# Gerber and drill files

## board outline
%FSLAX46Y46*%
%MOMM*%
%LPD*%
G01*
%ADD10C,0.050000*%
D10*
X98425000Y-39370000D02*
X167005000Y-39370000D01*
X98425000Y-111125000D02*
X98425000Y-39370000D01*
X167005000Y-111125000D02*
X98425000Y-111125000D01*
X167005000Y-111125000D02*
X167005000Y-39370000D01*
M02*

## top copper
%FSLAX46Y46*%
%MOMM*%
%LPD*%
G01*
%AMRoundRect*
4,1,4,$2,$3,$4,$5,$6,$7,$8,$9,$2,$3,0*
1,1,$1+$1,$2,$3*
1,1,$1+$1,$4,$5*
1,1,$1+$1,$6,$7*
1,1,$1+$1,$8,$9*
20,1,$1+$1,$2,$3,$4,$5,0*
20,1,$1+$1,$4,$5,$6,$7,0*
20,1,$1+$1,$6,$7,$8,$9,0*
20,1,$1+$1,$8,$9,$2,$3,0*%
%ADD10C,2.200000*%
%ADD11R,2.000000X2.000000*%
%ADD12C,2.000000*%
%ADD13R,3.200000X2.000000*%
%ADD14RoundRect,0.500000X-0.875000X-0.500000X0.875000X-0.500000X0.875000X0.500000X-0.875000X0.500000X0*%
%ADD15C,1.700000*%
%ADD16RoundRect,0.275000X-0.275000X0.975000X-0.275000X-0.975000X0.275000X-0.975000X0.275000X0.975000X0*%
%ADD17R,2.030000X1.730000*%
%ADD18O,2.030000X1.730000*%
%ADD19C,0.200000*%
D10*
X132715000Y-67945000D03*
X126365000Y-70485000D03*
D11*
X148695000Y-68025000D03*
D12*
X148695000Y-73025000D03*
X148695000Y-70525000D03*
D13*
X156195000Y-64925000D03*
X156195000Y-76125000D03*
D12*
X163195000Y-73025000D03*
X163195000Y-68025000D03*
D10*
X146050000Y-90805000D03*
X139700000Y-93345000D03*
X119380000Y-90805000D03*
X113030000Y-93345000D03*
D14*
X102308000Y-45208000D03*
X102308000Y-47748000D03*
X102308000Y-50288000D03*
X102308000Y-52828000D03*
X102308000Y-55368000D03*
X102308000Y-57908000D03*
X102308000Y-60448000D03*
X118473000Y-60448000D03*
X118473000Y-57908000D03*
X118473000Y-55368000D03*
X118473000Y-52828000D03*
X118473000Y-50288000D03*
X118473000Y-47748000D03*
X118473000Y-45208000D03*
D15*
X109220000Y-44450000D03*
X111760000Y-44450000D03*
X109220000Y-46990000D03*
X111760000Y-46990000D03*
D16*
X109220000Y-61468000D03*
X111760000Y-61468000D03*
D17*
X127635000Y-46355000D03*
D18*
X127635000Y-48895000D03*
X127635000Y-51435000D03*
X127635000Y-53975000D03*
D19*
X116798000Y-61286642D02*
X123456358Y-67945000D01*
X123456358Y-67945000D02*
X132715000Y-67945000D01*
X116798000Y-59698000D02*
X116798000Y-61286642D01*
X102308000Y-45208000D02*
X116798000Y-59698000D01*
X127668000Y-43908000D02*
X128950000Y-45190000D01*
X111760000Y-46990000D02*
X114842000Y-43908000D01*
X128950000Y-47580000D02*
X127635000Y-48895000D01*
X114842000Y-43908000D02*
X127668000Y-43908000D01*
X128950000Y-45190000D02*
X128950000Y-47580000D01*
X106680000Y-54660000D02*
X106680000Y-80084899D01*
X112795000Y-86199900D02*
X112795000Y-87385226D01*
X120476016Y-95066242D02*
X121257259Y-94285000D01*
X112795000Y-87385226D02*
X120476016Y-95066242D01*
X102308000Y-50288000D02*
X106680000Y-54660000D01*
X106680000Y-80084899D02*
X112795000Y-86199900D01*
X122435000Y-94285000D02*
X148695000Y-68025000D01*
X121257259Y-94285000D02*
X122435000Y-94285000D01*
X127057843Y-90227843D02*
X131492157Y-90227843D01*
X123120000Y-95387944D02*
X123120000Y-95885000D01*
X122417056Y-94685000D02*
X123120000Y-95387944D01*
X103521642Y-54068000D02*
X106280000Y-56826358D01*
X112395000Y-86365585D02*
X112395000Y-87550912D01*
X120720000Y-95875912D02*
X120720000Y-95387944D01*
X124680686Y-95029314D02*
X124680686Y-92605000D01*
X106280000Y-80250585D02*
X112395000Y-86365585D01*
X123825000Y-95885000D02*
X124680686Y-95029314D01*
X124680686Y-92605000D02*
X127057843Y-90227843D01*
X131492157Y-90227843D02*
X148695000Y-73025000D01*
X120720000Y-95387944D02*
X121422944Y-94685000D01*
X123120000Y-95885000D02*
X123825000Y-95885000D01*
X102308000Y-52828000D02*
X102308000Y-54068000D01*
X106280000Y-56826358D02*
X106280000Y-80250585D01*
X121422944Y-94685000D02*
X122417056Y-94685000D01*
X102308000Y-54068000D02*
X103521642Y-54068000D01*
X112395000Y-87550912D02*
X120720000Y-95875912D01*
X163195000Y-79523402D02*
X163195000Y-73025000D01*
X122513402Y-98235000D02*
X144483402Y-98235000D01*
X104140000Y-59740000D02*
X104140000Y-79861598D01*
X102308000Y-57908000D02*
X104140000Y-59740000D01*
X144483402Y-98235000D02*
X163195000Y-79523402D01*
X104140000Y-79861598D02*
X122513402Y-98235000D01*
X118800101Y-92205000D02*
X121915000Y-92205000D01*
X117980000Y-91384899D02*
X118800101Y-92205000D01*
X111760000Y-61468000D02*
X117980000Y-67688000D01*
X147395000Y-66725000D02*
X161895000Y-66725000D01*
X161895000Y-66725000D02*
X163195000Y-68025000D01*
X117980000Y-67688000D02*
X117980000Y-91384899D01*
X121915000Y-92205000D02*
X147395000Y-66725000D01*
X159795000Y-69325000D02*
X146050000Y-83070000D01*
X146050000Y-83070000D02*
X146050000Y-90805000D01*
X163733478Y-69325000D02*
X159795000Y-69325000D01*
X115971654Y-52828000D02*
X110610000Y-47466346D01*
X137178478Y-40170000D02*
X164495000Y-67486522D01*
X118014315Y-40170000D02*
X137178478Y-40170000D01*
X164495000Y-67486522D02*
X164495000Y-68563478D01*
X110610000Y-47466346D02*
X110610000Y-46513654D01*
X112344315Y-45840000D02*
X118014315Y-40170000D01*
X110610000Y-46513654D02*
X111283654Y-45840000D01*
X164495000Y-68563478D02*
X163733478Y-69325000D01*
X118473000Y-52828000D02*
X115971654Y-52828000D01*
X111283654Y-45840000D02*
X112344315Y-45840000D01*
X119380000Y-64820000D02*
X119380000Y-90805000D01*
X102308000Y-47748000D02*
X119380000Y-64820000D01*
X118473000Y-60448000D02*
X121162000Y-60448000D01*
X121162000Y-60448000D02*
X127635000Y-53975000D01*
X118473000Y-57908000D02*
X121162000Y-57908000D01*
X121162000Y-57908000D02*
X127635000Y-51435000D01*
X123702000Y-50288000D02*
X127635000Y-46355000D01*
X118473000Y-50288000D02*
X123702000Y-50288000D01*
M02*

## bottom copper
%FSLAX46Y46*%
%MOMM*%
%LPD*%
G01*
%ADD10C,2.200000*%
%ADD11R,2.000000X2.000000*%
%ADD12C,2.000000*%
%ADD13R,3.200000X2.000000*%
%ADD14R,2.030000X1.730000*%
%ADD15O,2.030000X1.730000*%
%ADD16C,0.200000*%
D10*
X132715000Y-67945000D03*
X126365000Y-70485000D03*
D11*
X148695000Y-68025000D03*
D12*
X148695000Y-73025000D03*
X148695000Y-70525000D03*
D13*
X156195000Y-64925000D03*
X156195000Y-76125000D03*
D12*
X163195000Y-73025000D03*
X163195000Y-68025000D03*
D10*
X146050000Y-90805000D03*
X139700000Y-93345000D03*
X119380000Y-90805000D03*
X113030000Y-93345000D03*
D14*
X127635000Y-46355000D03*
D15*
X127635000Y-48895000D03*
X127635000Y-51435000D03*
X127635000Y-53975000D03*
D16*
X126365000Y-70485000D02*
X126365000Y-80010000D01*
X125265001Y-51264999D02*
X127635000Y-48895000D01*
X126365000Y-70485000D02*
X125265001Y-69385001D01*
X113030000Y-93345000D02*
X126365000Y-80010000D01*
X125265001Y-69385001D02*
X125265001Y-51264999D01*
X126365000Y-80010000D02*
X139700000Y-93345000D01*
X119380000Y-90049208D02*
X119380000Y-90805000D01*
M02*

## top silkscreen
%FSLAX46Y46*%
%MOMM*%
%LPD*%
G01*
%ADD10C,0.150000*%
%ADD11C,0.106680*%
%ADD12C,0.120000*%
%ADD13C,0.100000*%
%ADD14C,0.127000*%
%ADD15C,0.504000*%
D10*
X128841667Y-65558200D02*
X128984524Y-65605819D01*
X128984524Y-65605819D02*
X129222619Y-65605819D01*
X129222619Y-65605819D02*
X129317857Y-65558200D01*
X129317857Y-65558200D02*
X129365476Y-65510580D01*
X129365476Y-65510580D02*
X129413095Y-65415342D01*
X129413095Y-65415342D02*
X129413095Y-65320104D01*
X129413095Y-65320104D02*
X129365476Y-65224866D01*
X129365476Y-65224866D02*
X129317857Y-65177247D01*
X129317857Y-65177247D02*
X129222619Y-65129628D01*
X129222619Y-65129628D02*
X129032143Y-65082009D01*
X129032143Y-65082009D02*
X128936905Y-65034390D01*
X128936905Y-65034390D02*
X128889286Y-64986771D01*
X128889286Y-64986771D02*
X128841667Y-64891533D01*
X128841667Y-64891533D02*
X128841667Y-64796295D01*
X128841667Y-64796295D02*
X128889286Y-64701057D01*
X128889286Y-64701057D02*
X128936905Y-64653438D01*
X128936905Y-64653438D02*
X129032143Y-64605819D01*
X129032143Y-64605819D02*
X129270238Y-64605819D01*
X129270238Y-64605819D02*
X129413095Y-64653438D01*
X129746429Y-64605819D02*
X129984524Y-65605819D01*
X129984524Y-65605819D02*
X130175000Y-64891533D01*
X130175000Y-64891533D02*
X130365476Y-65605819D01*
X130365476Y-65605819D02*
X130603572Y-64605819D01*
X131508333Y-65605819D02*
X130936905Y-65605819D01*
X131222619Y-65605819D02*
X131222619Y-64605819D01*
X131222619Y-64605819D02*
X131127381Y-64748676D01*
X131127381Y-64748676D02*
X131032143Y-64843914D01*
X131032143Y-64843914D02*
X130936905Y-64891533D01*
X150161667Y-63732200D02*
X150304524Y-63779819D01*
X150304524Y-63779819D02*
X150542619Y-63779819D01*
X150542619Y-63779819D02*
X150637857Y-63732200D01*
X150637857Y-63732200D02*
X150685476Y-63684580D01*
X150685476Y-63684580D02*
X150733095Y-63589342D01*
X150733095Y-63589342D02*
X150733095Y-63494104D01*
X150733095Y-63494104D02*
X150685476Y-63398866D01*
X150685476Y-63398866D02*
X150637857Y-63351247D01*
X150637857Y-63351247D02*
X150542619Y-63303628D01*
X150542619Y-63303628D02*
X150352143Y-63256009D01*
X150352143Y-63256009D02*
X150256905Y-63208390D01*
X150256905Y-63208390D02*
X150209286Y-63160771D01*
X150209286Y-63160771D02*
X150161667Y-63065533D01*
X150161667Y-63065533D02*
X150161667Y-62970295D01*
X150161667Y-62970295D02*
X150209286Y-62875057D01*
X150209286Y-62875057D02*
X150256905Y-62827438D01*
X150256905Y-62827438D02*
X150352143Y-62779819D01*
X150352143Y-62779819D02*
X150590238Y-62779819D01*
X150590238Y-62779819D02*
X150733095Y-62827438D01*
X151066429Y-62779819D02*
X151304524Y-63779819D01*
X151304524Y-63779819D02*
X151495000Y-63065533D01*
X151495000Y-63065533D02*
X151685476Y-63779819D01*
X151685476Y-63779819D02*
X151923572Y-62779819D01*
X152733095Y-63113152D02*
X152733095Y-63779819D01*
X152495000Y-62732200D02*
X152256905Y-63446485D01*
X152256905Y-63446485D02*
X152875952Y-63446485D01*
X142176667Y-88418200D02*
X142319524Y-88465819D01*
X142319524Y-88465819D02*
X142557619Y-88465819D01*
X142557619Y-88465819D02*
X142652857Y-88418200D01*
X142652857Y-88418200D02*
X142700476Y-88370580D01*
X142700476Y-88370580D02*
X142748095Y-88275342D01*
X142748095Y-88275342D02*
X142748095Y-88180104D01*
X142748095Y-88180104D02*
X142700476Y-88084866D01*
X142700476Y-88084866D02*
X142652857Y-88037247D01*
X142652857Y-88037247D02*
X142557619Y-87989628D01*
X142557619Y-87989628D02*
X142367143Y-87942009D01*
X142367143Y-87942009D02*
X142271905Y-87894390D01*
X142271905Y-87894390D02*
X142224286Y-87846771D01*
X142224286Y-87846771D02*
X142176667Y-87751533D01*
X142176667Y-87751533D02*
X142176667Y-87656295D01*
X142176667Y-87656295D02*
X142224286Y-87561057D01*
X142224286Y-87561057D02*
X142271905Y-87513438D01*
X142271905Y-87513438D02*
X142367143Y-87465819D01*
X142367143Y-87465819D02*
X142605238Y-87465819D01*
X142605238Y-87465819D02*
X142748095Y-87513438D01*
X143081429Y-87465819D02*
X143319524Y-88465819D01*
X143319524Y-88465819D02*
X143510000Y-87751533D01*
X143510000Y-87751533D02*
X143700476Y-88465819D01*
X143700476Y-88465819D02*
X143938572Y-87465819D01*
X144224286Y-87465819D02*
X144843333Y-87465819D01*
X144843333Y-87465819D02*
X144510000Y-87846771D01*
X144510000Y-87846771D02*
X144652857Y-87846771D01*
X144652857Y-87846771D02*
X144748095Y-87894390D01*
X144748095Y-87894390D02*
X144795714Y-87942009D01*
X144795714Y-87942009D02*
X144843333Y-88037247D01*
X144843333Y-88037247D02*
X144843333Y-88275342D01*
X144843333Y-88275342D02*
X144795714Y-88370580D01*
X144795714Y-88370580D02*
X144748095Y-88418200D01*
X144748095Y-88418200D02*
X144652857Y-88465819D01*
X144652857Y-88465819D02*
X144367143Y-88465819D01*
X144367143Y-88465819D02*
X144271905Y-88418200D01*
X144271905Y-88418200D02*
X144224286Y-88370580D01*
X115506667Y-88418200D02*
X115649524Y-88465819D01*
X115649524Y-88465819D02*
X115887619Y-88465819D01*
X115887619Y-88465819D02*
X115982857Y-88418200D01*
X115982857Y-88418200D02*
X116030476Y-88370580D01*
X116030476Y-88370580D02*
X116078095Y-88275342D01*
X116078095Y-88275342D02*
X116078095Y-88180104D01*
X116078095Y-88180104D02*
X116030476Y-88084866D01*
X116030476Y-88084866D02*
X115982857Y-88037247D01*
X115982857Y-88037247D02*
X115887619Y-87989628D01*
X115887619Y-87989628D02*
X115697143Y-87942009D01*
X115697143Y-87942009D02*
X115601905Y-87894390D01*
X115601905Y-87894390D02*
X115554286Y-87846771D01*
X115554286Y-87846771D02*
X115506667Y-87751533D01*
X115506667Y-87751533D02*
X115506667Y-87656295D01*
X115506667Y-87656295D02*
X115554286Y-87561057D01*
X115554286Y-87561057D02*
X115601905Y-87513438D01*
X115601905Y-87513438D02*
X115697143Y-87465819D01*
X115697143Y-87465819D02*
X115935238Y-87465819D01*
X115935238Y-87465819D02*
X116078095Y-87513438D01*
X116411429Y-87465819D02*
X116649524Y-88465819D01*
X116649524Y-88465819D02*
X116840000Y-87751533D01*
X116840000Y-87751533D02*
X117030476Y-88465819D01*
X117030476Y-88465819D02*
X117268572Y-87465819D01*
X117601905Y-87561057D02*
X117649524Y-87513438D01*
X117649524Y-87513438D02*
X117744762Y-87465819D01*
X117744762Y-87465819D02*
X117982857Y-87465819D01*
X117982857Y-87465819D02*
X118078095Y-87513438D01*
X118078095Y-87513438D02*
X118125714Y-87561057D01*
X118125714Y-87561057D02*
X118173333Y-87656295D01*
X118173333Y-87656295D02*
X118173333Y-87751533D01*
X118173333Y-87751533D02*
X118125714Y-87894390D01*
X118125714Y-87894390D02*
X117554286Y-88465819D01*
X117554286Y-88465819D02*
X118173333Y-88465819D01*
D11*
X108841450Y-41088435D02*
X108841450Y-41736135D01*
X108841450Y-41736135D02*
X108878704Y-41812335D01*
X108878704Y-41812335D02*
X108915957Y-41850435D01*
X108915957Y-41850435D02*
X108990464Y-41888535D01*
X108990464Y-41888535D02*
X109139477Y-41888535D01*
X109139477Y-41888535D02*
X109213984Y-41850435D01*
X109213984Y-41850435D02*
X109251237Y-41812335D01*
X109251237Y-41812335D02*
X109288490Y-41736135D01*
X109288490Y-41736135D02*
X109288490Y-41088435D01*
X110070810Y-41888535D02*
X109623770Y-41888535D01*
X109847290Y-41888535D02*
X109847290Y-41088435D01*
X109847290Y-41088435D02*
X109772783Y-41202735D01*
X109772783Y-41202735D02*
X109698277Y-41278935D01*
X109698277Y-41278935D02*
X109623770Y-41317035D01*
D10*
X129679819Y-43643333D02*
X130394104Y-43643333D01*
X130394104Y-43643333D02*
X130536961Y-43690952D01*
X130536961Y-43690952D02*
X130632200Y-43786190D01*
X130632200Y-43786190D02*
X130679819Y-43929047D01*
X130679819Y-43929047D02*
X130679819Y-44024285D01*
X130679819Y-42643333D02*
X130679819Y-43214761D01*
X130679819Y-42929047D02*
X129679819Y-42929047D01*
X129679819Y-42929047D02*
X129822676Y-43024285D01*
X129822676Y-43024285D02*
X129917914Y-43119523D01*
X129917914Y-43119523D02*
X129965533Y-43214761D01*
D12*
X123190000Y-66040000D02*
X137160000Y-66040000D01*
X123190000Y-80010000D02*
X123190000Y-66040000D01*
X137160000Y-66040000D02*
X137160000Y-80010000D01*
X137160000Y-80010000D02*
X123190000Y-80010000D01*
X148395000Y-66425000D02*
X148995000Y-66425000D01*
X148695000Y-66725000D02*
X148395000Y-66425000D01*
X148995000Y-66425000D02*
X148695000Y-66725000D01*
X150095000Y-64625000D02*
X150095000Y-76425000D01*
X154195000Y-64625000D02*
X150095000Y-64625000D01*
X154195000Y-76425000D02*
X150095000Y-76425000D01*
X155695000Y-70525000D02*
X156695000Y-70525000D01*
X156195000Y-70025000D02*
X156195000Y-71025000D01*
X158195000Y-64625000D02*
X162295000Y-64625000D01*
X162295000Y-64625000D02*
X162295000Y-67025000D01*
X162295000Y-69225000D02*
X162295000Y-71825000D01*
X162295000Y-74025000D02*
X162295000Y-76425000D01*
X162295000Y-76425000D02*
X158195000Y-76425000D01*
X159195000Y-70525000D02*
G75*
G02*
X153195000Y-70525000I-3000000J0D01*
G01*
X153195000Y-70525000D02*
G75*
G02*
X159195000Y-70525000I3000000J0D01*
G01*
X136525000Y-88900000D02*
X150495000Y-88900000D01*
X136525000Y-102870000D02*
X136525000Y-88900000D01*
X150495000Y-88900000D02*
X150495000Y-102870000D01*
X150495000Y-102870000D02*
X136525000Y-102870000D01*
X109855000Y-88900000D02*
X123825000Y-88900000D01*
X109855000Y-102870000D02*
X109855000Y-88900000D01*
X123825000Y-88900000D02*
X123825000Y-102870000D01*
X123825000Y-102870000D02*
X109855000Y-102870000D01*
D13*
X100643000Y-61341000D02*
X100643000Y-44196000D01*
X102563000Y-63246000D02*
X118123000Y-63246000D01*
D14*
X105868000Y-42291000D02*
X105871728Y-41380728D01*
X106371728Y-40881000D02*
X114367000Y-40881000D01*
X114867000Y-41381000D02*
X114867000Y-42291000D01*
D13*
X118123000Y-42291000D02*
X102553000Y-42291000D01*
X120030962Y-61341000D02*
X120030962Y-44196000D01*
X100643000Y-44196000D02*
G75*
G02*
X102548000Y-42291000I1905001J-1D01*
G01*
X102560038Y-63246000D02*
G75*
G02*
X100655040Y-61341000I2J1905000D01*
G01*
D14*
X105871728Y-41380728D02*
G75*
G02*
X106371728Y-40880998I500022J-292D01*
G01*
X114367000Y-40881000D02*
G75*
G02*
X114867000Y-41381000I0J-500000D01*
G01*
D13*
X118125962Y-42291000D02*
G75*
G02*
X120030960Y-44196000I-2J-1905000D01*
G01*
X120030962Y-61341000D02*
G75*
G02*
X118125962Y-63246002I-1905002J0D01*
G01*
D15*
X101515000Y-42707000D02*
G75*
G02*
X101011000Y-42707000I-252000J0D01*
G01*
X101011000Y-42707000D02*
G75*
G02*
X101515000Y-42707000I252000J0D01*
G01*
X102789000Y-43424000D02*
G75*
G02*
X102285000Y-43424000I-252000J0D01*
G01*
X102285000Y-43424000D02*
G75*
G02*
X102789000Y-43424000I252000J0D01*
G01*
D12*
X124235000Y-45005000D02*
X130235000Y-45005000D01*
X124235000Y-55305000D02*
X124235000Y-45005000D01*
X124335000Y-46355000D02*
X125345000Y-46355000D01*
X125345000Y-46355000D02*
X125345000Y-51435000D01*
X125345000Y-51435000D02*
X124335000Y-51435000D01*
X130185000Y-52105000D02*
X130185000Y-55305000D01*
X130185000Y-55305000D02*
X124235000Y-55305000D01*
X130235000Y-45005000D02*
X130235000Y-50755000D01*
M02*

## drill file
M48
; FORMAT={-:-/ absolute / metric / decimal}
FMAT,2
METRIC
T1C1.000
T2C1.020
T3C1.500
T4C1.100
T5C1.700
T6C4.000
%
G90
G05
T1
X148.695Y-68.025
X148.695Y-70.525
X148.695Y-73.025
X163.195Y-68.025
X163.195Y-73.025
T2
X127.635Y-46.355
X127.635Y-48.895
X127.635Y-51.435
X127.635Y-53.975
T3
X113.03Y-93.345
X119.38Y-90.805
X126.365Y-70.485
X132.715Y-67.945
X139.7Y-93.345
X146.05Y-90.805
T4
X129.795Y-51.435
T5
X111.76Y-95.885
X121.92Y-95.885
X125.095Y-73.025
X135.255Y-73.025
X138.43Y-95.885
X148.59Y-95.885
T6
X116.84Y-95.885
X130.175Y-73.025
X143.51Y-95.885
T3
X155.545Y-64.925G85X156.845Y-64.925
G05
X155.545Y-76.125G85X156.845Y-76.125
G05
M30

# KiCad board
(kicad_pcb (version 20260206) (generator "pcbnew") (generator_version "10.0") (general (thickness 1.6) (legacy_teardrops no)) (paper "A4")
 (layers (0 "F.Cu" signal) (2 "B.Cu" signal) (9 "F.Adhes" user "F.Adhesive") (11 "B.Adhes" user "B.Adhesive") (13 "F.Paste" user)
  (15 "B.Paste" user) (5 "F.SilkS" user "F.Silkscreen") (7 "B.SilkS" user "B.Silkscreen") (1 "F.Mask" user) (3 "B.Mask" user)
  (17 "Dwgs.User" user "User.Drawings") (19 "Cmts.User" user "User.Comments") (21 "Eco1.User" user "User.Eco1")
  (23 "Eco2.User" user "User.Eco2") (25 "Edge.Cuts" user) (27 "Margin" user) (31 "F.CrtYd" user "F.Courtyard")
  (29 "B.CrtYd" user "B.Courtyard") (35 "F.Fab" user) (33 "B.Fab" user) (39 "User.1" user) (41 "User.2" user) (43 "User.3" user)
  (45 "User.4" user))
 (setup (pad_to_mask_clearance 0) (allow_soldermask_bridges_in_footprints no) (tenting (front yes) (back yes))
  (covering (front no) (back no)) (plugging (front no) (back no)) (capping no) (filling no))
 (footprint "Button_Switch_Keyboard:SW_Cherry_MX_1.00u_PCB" (layer "F.Cu") (at 132.715 67.945)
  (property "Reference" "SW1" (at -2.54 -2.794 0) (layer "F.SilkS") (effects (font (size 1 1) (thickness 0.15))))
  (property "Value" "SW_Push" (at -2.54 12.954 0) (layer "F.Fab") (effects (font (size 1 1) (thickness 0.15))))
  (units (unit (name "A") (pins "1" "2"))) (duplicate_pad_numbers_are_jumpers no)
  (fp_line (start -9.525 -1.905) (end 4.445 -1.905) (stroke (width 0.12) (type solid)) (layer "F.SilkS"))
  (fp_line (start -9.525 12.065) (end -9.525 -1.905) (stroke (width 0.12) (type solid)) (layer "F.SilkS"))
  (fp_line (start 4.445 -1.905) (end 4.445 12.065) (stroke (width 0.12) (type solid)) (layer "F.SilkS"))
  (fp_line (start 4.445 12.065) (end -9.525 12.065) (stroke (width 0.12) (type solid)) (layer "F.SilkS"))
  (pad "" np_thru_hole circle (at -7.62 5.08) (size 1.7 1.7) (drill 1.7) (layers "*.Cu" "*.Mask"))
  (pad "" np_thru_hole circle (at -2.54 5.08) (size 4 4) (drill 4) (layers "*.Cu" "*.Mask"))
  (pad "" np_thru_hole circle (at 2.54 5.08) (size 1.7 1.7) (drill 1.7) (layers "*.Cu" "*.Mask"))
  (pad "1" thru_hole circle (at 0 0) (size 2.2 2.2) (drill 1.5) (layers "*.Cu" "*.Mask") (remove_unused_layers no) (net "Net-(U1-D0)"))
  (pad "2" thru_hole circle (at -6.35 2.54) (size 2.2 2.2) (drill 1.5) (layers "*.Cu" "*.Mask") (remove_unused_layers no)
   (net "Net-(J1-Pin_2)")))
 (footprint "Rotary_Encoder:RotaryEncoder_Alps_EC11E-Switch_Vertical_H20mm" (layer "F.Cu") (at 148.695 68.025)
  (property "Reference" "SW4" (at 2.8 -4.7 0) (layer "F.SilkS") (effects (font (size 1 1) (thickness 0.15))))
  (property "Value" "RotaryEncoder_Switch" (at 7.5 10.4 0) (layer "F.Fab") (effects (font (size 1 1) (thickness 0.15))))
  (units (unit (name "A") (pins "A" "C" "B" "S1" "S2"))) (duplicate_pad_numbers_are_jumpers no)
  (fp_line (start -0.3 -1.6) (end 0.3 -1.6) (stroke (width 0.12) (type solid)) (layer "F.SilkS"))
  (fp_line (start 0 -1.3) (end -0.3 -1.6) (stroke (width 0.12) (type solid)) (layer "F.SilkS"))
  (fp_line (start 0.3 -1.6) (end 0 -1.3) (stroke (width 0.12) (type solid)) (layer "F.SilkS"))
  (fp_line (start 1.4 -3.4) (end 1.4 8.4) (stroke (width 0.12) (type solid)) (layer "F.SilkS"))
  (fp_line (start 5.5 -3.4) (end 1.4 -3.4) (stroke (width 0.12) (type solid)) (layer "F.SilkS"))
  (fp_line (start 5.5 8.4) (end 1.4 8.4) (stroke (width 0.12) (type solid)) (layer "F.SilkS"))
  (fp_line (start 7 2.5) (end 8 2.5) (stroke (width 0.12) (type solid)) (layer "F.SilkS"))
  (fp_line (start 7.5 2) (end 7.5 3) (stroke (width 0.12) (type solid)) (layer "F.SilkS"))
  (fp_line (start 9.5 -3.4) (end 13.6 -3.4) (stroke (width 0.12) (type solid)) (layer "F.SilkS"))
  (fp_line (start 13.6 -3.4) (end 13.6 -1) (stroke (width 0.12) (type solid)) (layer "F.SilkS"))
  (fp_line (start 13.6 1.2) (end 13.6 3.8) (stroke (width 0.12) (type solid)) (layer "F.SilkS"))
  (fp_line (start 13.6 6) (end 13.6 8.4) (stroke (width 0.12) (type solid)) (layer "F.SilkS"))
  (fp_line (start 13.6 8.4) (end 9.5 8.4) (stroke (width 0.12) (type solid)) (layer "F.SilkS"))
  (fp_circle (center 7.5 2.5) (end 10.5 2.5) (stroke (width 0.12) (type solid)) (fill no) (layer "F.SilkS"))
  (pad "A" thru_hole rect (at 0 0) (size 2 2) (drill 1) (layers "*.Cu" "*.Mask") (remove_unused_layers no) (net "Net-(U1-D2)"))
  (pad "B" thru_hole circle (at 0 5) (size 2 2) (drill 1) (layers "*.Cu" "*.Mask") (remove_unused_layers no) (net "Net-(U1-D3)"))
  (pad "C" thru_hole circle (at 0 2.5) (size 2 2) (drill 1) (layers "*.Cu" "*.Mask") (remove_unused_layers no)
   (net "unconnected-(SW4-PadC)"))
  (pad "MP" thru_hole rect (at 7.5 -3.1) (size 3.2 2) (drill oval 2.8 1.5) (layers "*.Cu" "*.Mask") (remove_unused_layers no))
  (pad "MP" thru_hole rect (at 7.5 8.1) (size 3.2 2) (drill oval 2.8 1.5) (layers "*.Cu" "*.Mask") (remove_unused_layers no))
  (pad "S1" thru_hole circle (at 14.5 5) (size 2 2) (drill 1) (layers "*.Cu" "*.Mask") (remove_unused_layers no) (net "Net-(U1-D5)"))
  (pad "S2" thru_hole circle (at 14.5 0) (size 2 2) (drill 1) (layers "*.Cu" "*.Mask") (remove_unused_layers no) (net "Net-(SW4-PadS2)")))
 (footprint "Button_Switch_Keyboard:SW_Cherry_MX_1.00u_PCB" (layer "F.Cu") (at 146.05 90.805)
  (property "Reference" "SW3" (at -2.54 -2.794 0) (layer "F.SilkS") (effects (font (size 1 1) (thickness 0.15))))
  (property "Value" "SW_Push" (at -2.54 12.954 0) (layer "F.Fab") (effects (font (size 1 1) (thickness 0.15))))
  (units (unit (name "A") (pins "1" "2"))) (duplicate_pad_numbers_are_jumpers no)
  (fp_line (start -9.525 -1.905) (end 4.445 -1.905) (stroke (width 0.12) (type solid)) (layer "F.SilkS"))
  (fp_line (start -9.525 12.065) (end -9.525 -1.905) (stroke (width 0.12) (type solid)) (layer "F.SilkS"))
  (fp_line (start 4.445 -1.905) (end 4.445 12.065) (stroke (width 0.12) (type solid)) (layer "F.SilkS"))
  (fp_line (start 4.445 12.065) (end -9.525 12.065) (stroke (width 0.12) (type solid)) (layer "F.SilkS"))
  (pad "" np_thru_hole circle (at -7.62 5.08) (size 1.7 1.7) (drill 1.7) (layers "*.Cu" "*.Mask"))
  (pad "" np_thru_hole circle (at -2.54 5.08) (size 4 4) (drill 4) (layers "*.Cu" "*.Mask"))
  (pad "" np_thru_hole circle (at 2.54 5.08) (size 1.7 1.7) (drill 1.7) (layers "*.Cu" "*.Mask"))
  (pad "1" thru_hole circle (at 0 0) (size 2.2 2.2) (drill 1.5) (layers "*.Cu" "*.Mask") (remove_unused_layers no) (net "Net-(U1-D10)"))
  (pad "2" thru_hole circle (at -6.35 2.54) (size 2.2 2.2) (drill 1.5) (layers "*.Cu" "*.Mask") (remove_unused_layers no)
   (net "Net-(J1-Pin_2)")))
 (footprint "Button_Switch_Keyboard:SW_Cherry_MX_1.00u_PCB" (layer "F.Cu") (at 119.38 90.805)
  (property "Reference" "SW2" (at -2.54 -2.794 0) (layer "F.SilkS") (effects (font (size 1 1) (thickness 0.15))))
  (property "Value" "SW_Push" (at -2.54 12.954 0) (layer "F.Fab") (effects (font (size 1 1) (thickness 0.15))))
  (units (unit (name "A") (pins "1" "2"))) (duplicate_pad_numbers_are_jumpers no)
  (fp_line (start -9.525 -1.905) (end 4.445 -1.905) (stroke (width 0.12) (type solid)) (layer "F.SilkS"))
  (fp_line (start -9.525 12.065) (end -9.525 -1.905) (stroke (width 0.12) (type solid)) (layer "F.SilkS"))
  (fp_line (start 4.445 -1.905) (end 4.445 12.065) (stroke (width 0.12) (type solid)) (layer "F.SilkS"))
  (fp_line (start 4.445 12.065) (end -9.525 12.065) (stroke (width 0.12) (type solid)) (layer "F.SilkS"))
  (pad "" np_thru_hole circle (at -7.62 5.08) (size 1.7 1.7) (drill 1.7) (layers "*.Cu" "*.Mask"))
  (pad "" np_thru_hole circle (at -2.54 5.08) (size 4 4) (drill 4) (layers "*.Cu" "*.Mask"))
  (pad "" np_thru_hole circle (at 2.54 5.08) (size 1.7 1.7) (drill 1.7) (layers "*.Cu" "*.Mask"))
  (pad "1" thru_hole circle (at 0 0) (size 2.2 2.2) (drill 1.5) (layers "*.Cu" "*.Mask") (remove_unused_layers no) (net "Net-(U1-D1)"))
  (pad "2" thru_hole circle (at -6.35 2.54) (size 2.2 2.2) (drill 1.5) (layers "*.Cu" "*.Mask") (remove_unused_layers no)
   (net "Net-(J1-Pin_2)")))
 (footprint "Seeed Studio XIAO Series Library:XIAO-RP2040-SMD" (layer "F.Cu") (at 101.473 63.328)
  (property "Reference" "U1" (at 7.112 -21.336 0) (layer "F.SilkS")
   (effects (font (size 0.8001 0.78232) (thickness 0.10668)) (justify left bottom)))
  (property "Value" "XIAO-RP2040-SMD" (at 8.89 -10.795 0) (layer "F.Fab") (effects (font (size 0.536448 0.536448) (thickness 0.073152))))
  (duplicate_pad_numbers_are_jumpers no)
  (fp_line (start -0.83 -1.987) (end -0.83 -19.132) (stroke (width 0.1) (type solid)) (layer "F.SilkS"))
  (fp_line (start 1.09 -0.082) (end 16.65 -0.082) (stroke (width 0.1) (type solid)) (layer "F.SilkS"))
  (fp_line (start 4.395 -21.037) (end 4.398728 -21.947272) (stroke (width 0.127) (type solid)) (layer "F.SilkS"))
  (fp_line (start 4.898728 -22.447) (end 12.894 -22.447) (stroke (width 0.127) (type solid)) (layer "F.SilkS"))
  (fp_line (start 13.394 -21.947) (end 13.394 -21.037) (stroke (width 0.127) (type solid)) (layer "F.SilkS"))
  (fp_line (start 16.65 -21.037) (end 1.08 -21.037) (stroke (width 0.1) (type solid)) (layer "F.SilkS"))
  (fp_line (start 18.557962 -1.987) (end 18.557962 -19.132) (stroke (width 0.1) (type solid)) (layer "F.SilkS"))
  (fp_arc (start -0.83 -19.132) (mid -0.272038 -20.479038) (end 1.075 -21.037) (stroke (width 0.1) (type solid)) (layer "F.SilkS"))
  (fp_arc (start 1.087038 -0.082) (mid -0.26 -0.639962) (end -0.817962 -1.987) (stroke (width 0.1) (type solid)) (layer "F.SilkS"))
  (fp_arc (start 4.398728 -21.947272) (mid 4.545276 -22.300644) (end 4.898728 -22.447) (stroke (width 0.127) (type default))
   (layer "F.SilkS"))
  (fp_arc (start 12.894 -22.447) (mid 13.247553 -22.300553) (end 13.394 -21.947) (stroke (width 0.127) (type default)) (layer "F.SilkS"))
  (fp_arc (start 16.652962 -21.037) (mid 18 -20.479038) (end 18.557962 -19.132) (stroke (width 0.1) (type solid)) (layer "F.SilkS"))
  (fp_arc (start 18.557962 -1.987) (mid 18 -0.639962) (end 16.652962 -0.082) (stroke (width 0.1) (type solid)) (layer "F.SilkS"))
  (fp_circle (center -0.21 -20.621) (end -0.21 -20.875) (stroke (width 0.5) (type solid)) (fill yes) (layer "F.SilkS"))
  (fp_circle (center 1.064 -19.904) (end 1.064 -20.158) (stroke (width 0.5) (type solid)) (fill yes) (layer "F.SilkS"))
  (pad "1" smd roundrect (at 0.835 -18.12) (size 2.75 2) (layers "F.Cu" "F.Mask" "F.Paste") (roundrect_rratio 0.25) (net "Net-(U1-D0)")
   (solder_mask_margin 0.0508) (thermal_bridge_angle 45))
  (pad "2" smd roundrect (at 0.835 -15.58) (size 2.75 2) (layers "F.Cu" "F.Mask" "F.Paste") (roundrect_rratio 0.25) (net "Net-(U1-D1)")
   (solder_mask_margin 0.0508) (thermal_bridge_angle 45))
  (pad "3" smd roundrect (at 0.835 -13.04) (size 2.75 2) (layers "F.Cu" "F.Mask" "F.Paste") (roundrect_rratio 0.25) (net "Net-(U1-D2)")
   (solder_mask_margin 0.0508) (thermal_bridge_angle 45))
  (pad "4" smd roundrect (at 0.835 -10.5) (size 2.75 2) (layers "F.Cu" "F.Mask" "F.Paste") (roundrect_rratio 0.25) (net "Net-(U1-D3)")
   (solder_mask_margin 0.0508) (thermal_bridge_angle 45))
  (pad "5" smd roundrect (at 0.835 -7.96) (size 2.75 2) (layers "F.Cu" "F.Mask" "F.Paste") (roundrect_rratio 0.25)
   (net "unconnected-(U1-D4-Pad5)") (solder_mask_margin 0.0508) (thermal_bridge_angle 45))
  (pad "6" smd roundrect (at 0.835 -5.42) (size 2.75 2) (layers "F.Cu" "F.Mask" "F.Paste") (roundrect_rratio 0.25) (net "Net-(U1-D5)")
   (solder_mask_margin 0.0508) (thermal_bridge_angle 45))
  (pad "7" smd roundrect (at 0.835 -2.88) (size 2.75 2) (layers "F.Cu" "F.Mask" "F.Paste") (roundrect_rratio 0.25)
   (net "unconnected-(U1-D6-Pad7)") (solder_mask_margin 0.0508) (thermal_bridge_angle 45))
  (pad "8" smd roundrect (at 17 -2.88) (size 2.75 2) (layers "F.Cu" "F.Mask" "F.Paste") (roundrect_rratio 0.25) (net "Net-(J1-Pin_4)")
   (solder_mask_margin 0.0508) (thermal_bridge_angle 45))
  (pad "9" smd roundrect (at 17 -5.42) (size 2.75 2) (layers "F.Cu" "F.Mask" "F.Paste") (roundrect_rratio 0.25) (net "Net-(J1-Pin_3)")
   (solder_mask_margin 0.0508) (thermal_bridge_angle 45))
  (pad "10" smd roundrect (at 17 -7.96) (size 2.75 2) (layers "F.Cu" "F.Mask" "F.Paste") (roundrect_rratio 0.25)
   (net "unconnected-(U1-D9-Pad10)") (solder_mask_margin 0.0508) (thermal_bridge_angle 45))
  (pad "11" smd roundrect (at 17 -10.5) (size 2.75 2) (layers "F.Cu" "F.Mask" "F.Paste") (roundrect_rratio 0.25) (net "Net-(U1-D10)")
   (solder_mask_margin 0.0508) (thermal_bridge_angle 45))
  (pad "12" smd roundrect (at 17 -13.04) (size 2.75 2) (layers "F.Cu" "F.Mask" "F.Paste") (roundrect_rratio 0.25) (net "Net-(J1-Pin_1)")
   (solder_mask_margin 0.0508) (thermal_bridge_angle 45))
  (pad "13" smd roundrect (at 17 -15.58) (size 2.75 2) (layers "F.Cu" "F.Mask" "F.Paste") (roundrect_rratio 0.25)
   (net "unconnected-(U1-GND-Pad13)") (solder_mask_margin 0.0508) (thermal_bridge_angle 45))
  (pad "14" smd roundrect (at 17 -18.12) (size 2.75 2) (layers "F.Cu" "F.Mask" "F.Paste") (roundrect_rratio 0.25)
   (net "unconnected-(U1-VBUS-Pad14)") (solder_mask_margin 0.0508) (thermal_bridge_angle 45))
  (pad "15" smd circle (at 7.747 -18.878) (size 1.7 1.7) (layers "F.Cu" "F.Mask" "F.Paste") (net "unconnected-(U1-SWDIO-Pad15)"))
  (pad "16" smd circle (at 10.287 -18.878) (size 1.7 1.7) (layers "F.Cu" "F.Mask" "F.Paste") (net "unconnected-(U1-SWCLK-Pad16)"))
  (pad "17" smd circle (at 7.747 -16.338) (size 1.7 1.7) (layers "F.Cu" "F.Mask" "F.Paste") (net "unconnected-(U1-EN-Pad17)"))
  (pad "18" smd circle (at 10.287 -16.338) (size 1.7 1.7) (layers "F.Cu" "F.Mask" "F.Paste") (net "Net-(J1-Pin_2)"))
  (pad "19" smd roundrect (at 7.747 -1.86 270) (size 2.5 1.1) (layers "F.Cu" "F.Mask" "F.Paste") (roundrect_rratio 0.25)
   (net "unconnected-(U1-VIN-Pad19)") (thermal_bridge_angle 45))
  (pad "20" smd roundrect (at 10.287 -1.86 270) (size 2.5 1.1) (layers "F.Cu" "F.Mask" "F.Paste") (roundrect_rratio 0.25)
   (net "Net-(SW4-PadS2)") (thermal_bridge_angle 45)))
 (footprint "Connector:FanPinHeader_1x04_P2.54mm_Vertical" (layer "F.Cu") (at 127.635 46.355 -90)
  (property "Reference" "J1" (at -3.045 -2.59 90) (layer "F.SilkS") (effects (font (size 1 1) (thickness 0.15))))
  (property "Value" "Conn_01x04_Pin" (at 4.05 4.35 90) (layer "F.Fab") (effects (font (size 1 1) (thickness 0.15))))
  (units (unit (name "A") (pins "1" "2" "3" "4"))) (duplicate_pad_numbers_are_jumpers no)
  (fp_line (start -1.35 3.4) (end -1.35 -2.6) (stroke (width 0.12) (type solid)) (layer "F.SilkS"))
  (fp_line (start 8.95 3.4) (end -1.35 3.4) (stroke (width 0.12) (type solid)) (layer "F.SilkS"))
  (fp_line (start 0 3.3) (end 0 2.29) (stroke (width 0.12) (type solid)) (layer "F.SilkS"))
  (fp_line (start 0 2.29) (end 5.08 2.29) (stroke (width 0.12) (type solid)) (layer "F.SilkS"))
  (fp_line (start 5.08 2.29) (end 5.08 3.3) (stroke (width 0.12) (type solid)) (layer "F.SilkS"))
  (fp_line (start 5.75 -2.55) (end 8.95 -2.55) (stroke (width 0.12) (type solid)) (layer "F.SilkS"))
  (fp_line (start 8.95 -2.55) (end 8.95 3.4) (stroke (width 0.12) (type solid)) (layer "F.SilkS"))
  (fp_line (start -1.35 -2.6) (end 4.4 -2.6) (stroke (width 0.12) (type solid)) (layer "F.SilkS"))
  (pad "" np_thru_hole circle (at 5.08 -2.16) (size 1.1 1.1) (drill 1.1) (layers "*.Cu" "*.Mask"))
  (pad "1" thru_hole rect (at 0 0) (size 2.03 1.73) (drill 1.02) (layers "*.Cu" "*.Mask") (remove_unused_layers no) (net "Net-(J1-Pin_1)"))
  (pad "2" thru_hole oval (at 2.54 0) (size 2.03 1.73) (drill 1.02) (layers "*.Cu" "*.Mask") (remove_unused_layers no)
   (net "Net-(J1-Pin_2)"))
  (pad "3" thru_hole oval (at 5.08 0) (size 2.03 1.73) (drill 1.02) (layers "*.Cu" "*.Mask") (remove_unused_layers no)
   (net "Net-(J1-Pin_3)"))
  (pad "4" thru_hole oval (at 7.62 0) (size 2.03 1.73) (drill 1.02) (layers "*.Cu" "*.Mask") (remove_unused_layers no)
   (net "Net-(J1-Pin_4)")))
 (gr_line (start 98.425 39.37) (end 167.005 39.37) (stroke (width 0.05) (type default)) (layer "Edge.Cuts"))
 (gr_line (start 98.425 111.125) (end 98.425 39.37) (stroke (width 0.05) (type default)) (layer "Edge.Cuts"))
 (gr_line (start 167.005 111.125) (end 98.425 111.125) (stroke (width 0.05) (type default)) (layer "Edge.Cuts"))
 (gr_line (start 167.005 111.125) (end 167.005 39.37) (stroke (width 0.05) (type default)) (layer "Edge.Cuts"))
 (segment (start 116.798 61.286642) (end 123.456358 67.945) (width 0.2) (layer "F.Cu") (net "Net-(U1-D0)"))
 (segment (start 123.456358 67.945) (end 132.715 67.945) (width 0.2) (layer "F.Cu") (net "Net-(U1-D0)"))
 (segment (start 116.798 59.698) (end 116.798 61.286642) (width 0.2) (layer "F.Cu") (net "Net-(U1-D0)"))
 (segment (start 102.308 45.208) (end 116.798 59.698) (width 0.2) (layer "F.Cu") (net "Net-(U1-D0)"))
 (segment (start 127.668 43.908) (end 128.95 45.19) (width 0.2) (layer "F.Cu") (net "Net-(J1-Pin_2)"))
 (segment (start 111.76 46.99) (end 114.842 43.908) (width 0.2) (layer "F.Cu") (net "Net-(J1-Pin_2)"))
 (segment (start 128.95 47.58) (end 127.635 48.895) (width 0.2) (layer "F.Cu") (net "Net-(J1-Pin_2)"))
 (segment (start 114.842 43.908) (end 127.668 43.908) (width 0.2) (layer "F.Cu") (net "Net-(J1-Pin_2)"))
 (segment (start 128.95 45.19) (end 128.95 47.58) (width 0.2) (layer "F.Cu") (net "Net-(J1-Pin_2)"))
 (segment (start 126.365 70.485) (end 126.365 80.01) (width 0.2) (layer "B.Cu") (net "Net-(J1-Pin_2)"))
 (segment (start 125.265001 51.264999) (end 127.635 48.895) (width 0.2) (layer "B.Cu") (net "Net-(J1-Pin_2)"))
 (segment (start 126.365 70.485) (end 125.265001 69.385001) (width 0.2) (layer "B.Cu") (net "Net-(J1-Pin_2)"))
 (segment (start 113.03 93.345) (end 126.365 80.01) (width 0.2) (layer "B.Cu") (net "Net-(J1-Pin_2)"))
 (segment (start 125.265001 69.385001) (end 125.265001 51.264999) (width 0.2) (layer "B.Cu") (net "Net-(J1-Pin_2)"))
 (segment (start 126.365 80.01) (end 139.7 93.345) (width 0.2) (layer "B.Cu") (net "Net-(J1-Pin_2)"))
 (segment (start 106.68 54.66) (end 106.68 80.084899) (width 0.2) (layer "F.Cu") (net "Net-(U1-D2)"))
 (segment (start 112.795 86.1999) (end 112.795 87.385226) (width 0.2) (layer "F.Cu") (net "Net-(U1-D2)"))
 (segment (start 120.476016 95.066242) (end 121.257259 94.285) (width 0.2) (layer "F.Cu") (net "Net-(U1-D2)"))
 (segment (start 112.795 87.385226) (end 120.476016 95.066242) (width 0.2) (layer "F.Cu") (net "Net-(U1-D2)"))
 (segment (start 102.308 50.288) (end 106.68 54.66) (width 0.2) (layer "F.Cu") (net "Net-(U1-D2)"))
 (segment (start 106.68 80.084899) (end 112.795 86.1999) (width 0.2) (layer "F.Cu") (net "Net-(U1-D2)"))
 (segment (start 122.435 94.285) (end 148.695 68.025) (width 0.2) (layer "F.Cu") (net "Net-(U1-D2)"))
 (segment (start 121.257259 94.285) (end 122.435 94.285) (width 0.2) (layer "F.Cu") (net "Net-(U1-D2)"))
 (segment (start 127.057843 90.227843) (end 131.492157 90.227843) (width 0.2) (layer "F.Cu") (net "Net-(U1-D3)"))
 (segment (start 123.12 95.387944) (end 123.12 95.885) (width 0.2) (layer "F.Cu") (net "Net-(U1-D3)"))
 (segment (start 122.417056 94.685) (end 123.12 95.387944) (width 0.2) (layer "F.Cu") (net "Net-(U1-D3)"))
 (segment (start 103.521642 54.068) (end 106.28 56.826358) (width 0.2) (layer "F.Cu") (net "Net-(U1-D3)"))
 (segment (start 112.395 86.365585) (end 112.395 87.550912) (width 0.2) (layer "F.Cu") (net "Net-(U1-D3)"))
 (segment (start 120.72 95.875912) (end 120.72 95.387944) (width 0.2) (layer "F.Cu") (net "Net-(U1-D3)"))
 (segment (start 124.680686 95.029314) (end 124.680686 92.605) (width 0.2) (layer "F.Cu") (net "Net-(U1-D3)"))
 (segment (start 106.28 80.250585) (end 112.395 86.365585) (width 0.2) (layer "F.Cu") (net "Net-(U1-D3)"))
 (segment (start 123.825 95.885) (end 124.680686 95.029314) (width 0.2) (layer "F.Cu") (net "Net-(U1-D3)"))
 (segment (start 124.680686 92.605) (end 127.057843 90.227843) (width 0.2) (layer "F.Cu") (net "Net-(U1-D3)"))
 (segment (start 131.492157 90.227843) (end 148.695 73.025) (width 0.2) (layer "F.Cu") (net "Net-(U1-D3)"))
 (segment (start 120.72 95.387944) (end 121.422944 94.685) (width 0.2) (layer "F.Cu") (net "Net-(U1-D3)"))
 (segment (start 123.12 95.885) (end 123.825 95.885) (width 0.2) (layer "F.Cu") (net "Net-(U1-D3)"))
 (segment (start 102.308 52.828) (end 102.308 54.068) (width 0.2) (layer "F.Cu") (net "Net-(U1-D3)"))
 (segment (start 106.28 56.826358) (end 106.28 80.250585) (width 0.2) (layer "F.Cu") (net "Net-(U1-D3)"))
 (segment (start 121.422944 94.685) (end 122.417056 94.685) (width 0.2) (layer "F.Cu") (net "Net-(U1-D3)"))
 (segment (start 102.308 54.068) (end 103.521642 54.068) (width 0.2) (layer "F.Cu") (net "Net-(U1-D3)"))
 (segment (start 112.395 87.550912) (end 120.72 95.875912) (width 0.2) (layer "F.Cu") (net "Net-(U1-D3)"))
 (segment (start 163.195 79.523402) (end 163.195 73.025) (width 0.2) (layer "F.Cu") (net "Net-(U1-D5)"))
 (segment (start 122.513402 98.235) (end 144.483402 98.235) (width 0.2) (layer "F.Cu") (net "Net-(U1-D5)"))
 (segment (start 104.14 59.74) (end 104.14 79.861598) (width 0.2) (layer "F.Cu") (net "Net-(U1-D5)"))
 (segment (start 102.308 57.908) (end 104.14 59.74) (width 0.2) (layer "F.Cu") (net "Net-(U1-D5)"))
 (segment (start 144.483402 98.235) (end 163.195 79.523402) (width 0.2) (layer "F.Cu") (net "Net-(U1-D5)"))
 (segment (start 104.14 79.861598) (end 122.513402 98.235) (width 0.2) (layer "F.Cu") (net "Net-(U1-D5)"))
 (segment (start 118.800101 92.205) (end 121.915 92.205) (width 0.2) (layer "F.Cu") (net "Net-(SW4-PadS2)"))
 (segment (start 117.98 91.384899) (end 118.800101 92.205) (width 0.2) (layer "F.Cu") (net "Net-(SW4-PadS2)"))
 (segment (start 111.76 61.468) (end 117.98 67.688) (width 0.2) (layer "F.Cu") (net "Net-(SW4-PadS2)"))
 (segment (start 147.395 66.725) (end 161.895 66.725) (width 0.2) (layer "F.Cu") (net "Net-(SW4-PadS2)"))
 (segment (start 161.895 66.725) (end 163.195 68.025) (width 0.2) (layer "F.Cu") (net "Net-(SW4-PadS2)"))
 (segment (start 117.98 67.688) (end 117.98 91.384899) (width 0.2) (layer "F.Cu") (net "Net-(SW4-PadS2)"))
 (segment (start 121.915 92.205) (end 147.395 66.725) (width 0.2) (layer "F.Cu") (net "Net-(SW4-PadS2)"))
 (segment (start 159.795 69.325) (end 146.05 83.07) (width 0.2) (layer "F.Cu") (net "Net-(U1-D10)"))
 (segment (start 146.05 83.07) (end 146.05 90.805) (width 0.2) (layer "F.Cu") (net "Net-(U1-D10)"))
 (segment (start 163.733478 69.325) (end 159.795 69.325) (width 0.2) (layer "F.Cu") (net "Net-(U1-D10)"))
 (segment (start 115.971654 52.828) (end 110.61 47.466346) (width 0.2) (layer "F.Cu") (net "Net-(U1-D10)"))
 (segment (start 137.178478 40.17) (end 164.495 67.486522) (width 0.2) (layer "F.Cu") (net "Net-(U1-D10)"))
 (segment (start 118.014315 40.17) (end 137.178478 40.17) (width 0.2) (layer "F.Cu") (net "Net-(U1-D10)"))
 (segment (start 164.495 67.486522) (end 164.495 68.563478) (width 0.2) (layer "F.Cu") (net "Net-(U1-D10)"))
 (segment (start 110.61 47.466346) (end 110.61 46.513654) (width 0.2) (layer "F.Cu") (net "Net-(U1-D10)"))
 (segment (start 112.344315 45.84) (end 118.014315 40.17) (width 0.2) (layer "F.Cu") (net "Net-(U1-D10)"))
 (segment (start 110.61 46.513654) (end 111.283654 45.84) (width 0.2) (layer "F.Cu") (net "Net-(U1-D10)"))
 (segment (start 164.495 68.563478) (end 163.733478 69.325) (width 0.2) (layer "F.Cu") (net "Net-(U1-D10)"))
 (segment (start 118.473 52.828) (end 115.971654 52.828) (width 0.2) (layer "F.Cu") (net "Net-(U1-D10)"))
 (segment (start 111.283654 45.84) (end 112.344315 45.84) (width 0.2) (layer "F.Cu") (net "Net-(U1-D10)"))
 (segment (start 119.38 64.82) (end 119.38 90.805) (width 0.2) (layer "F.Cu") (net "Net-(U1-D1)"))
 (segment (start 102.308 47.748) (end 119.38 64.82) (width 0.2) (layer "F.Cu") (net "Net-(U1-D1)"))
 (segment (start 119.38 90.049208) (end 119.38 90.805) (width 0.2) (layer "B.Cu") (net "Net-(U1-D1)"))
 (segment (start 118.473 60.448) (end 121.162 60.448) (width 0.2) (layer "F.Cu") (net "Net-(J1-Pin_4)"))
 (segment (start 121.162 60.448) (end 127.635 53.975) (width 0.2) (layer "F.Cu") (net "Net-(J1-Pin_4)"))
 (segment (start 118.473 57.908) (end 121.162 57.908) (width 0.2) (layer "F.Cu") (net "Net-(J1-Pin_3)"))
 (segment (start 121.162 57.908) (end 127.635 51.435) (width 0.2) (layer "F.Cu") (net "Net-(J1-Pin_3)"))
 (segment (start 123.702 50.288) (end 127.635 46.355) (width 0.2) (layer "F.Cu") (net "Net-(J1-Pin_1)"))
 (segment (start 118.473 50.288) (end 123.702 50.288) (width 0.2) (layer "F.Cu") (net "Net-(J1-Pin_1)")))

